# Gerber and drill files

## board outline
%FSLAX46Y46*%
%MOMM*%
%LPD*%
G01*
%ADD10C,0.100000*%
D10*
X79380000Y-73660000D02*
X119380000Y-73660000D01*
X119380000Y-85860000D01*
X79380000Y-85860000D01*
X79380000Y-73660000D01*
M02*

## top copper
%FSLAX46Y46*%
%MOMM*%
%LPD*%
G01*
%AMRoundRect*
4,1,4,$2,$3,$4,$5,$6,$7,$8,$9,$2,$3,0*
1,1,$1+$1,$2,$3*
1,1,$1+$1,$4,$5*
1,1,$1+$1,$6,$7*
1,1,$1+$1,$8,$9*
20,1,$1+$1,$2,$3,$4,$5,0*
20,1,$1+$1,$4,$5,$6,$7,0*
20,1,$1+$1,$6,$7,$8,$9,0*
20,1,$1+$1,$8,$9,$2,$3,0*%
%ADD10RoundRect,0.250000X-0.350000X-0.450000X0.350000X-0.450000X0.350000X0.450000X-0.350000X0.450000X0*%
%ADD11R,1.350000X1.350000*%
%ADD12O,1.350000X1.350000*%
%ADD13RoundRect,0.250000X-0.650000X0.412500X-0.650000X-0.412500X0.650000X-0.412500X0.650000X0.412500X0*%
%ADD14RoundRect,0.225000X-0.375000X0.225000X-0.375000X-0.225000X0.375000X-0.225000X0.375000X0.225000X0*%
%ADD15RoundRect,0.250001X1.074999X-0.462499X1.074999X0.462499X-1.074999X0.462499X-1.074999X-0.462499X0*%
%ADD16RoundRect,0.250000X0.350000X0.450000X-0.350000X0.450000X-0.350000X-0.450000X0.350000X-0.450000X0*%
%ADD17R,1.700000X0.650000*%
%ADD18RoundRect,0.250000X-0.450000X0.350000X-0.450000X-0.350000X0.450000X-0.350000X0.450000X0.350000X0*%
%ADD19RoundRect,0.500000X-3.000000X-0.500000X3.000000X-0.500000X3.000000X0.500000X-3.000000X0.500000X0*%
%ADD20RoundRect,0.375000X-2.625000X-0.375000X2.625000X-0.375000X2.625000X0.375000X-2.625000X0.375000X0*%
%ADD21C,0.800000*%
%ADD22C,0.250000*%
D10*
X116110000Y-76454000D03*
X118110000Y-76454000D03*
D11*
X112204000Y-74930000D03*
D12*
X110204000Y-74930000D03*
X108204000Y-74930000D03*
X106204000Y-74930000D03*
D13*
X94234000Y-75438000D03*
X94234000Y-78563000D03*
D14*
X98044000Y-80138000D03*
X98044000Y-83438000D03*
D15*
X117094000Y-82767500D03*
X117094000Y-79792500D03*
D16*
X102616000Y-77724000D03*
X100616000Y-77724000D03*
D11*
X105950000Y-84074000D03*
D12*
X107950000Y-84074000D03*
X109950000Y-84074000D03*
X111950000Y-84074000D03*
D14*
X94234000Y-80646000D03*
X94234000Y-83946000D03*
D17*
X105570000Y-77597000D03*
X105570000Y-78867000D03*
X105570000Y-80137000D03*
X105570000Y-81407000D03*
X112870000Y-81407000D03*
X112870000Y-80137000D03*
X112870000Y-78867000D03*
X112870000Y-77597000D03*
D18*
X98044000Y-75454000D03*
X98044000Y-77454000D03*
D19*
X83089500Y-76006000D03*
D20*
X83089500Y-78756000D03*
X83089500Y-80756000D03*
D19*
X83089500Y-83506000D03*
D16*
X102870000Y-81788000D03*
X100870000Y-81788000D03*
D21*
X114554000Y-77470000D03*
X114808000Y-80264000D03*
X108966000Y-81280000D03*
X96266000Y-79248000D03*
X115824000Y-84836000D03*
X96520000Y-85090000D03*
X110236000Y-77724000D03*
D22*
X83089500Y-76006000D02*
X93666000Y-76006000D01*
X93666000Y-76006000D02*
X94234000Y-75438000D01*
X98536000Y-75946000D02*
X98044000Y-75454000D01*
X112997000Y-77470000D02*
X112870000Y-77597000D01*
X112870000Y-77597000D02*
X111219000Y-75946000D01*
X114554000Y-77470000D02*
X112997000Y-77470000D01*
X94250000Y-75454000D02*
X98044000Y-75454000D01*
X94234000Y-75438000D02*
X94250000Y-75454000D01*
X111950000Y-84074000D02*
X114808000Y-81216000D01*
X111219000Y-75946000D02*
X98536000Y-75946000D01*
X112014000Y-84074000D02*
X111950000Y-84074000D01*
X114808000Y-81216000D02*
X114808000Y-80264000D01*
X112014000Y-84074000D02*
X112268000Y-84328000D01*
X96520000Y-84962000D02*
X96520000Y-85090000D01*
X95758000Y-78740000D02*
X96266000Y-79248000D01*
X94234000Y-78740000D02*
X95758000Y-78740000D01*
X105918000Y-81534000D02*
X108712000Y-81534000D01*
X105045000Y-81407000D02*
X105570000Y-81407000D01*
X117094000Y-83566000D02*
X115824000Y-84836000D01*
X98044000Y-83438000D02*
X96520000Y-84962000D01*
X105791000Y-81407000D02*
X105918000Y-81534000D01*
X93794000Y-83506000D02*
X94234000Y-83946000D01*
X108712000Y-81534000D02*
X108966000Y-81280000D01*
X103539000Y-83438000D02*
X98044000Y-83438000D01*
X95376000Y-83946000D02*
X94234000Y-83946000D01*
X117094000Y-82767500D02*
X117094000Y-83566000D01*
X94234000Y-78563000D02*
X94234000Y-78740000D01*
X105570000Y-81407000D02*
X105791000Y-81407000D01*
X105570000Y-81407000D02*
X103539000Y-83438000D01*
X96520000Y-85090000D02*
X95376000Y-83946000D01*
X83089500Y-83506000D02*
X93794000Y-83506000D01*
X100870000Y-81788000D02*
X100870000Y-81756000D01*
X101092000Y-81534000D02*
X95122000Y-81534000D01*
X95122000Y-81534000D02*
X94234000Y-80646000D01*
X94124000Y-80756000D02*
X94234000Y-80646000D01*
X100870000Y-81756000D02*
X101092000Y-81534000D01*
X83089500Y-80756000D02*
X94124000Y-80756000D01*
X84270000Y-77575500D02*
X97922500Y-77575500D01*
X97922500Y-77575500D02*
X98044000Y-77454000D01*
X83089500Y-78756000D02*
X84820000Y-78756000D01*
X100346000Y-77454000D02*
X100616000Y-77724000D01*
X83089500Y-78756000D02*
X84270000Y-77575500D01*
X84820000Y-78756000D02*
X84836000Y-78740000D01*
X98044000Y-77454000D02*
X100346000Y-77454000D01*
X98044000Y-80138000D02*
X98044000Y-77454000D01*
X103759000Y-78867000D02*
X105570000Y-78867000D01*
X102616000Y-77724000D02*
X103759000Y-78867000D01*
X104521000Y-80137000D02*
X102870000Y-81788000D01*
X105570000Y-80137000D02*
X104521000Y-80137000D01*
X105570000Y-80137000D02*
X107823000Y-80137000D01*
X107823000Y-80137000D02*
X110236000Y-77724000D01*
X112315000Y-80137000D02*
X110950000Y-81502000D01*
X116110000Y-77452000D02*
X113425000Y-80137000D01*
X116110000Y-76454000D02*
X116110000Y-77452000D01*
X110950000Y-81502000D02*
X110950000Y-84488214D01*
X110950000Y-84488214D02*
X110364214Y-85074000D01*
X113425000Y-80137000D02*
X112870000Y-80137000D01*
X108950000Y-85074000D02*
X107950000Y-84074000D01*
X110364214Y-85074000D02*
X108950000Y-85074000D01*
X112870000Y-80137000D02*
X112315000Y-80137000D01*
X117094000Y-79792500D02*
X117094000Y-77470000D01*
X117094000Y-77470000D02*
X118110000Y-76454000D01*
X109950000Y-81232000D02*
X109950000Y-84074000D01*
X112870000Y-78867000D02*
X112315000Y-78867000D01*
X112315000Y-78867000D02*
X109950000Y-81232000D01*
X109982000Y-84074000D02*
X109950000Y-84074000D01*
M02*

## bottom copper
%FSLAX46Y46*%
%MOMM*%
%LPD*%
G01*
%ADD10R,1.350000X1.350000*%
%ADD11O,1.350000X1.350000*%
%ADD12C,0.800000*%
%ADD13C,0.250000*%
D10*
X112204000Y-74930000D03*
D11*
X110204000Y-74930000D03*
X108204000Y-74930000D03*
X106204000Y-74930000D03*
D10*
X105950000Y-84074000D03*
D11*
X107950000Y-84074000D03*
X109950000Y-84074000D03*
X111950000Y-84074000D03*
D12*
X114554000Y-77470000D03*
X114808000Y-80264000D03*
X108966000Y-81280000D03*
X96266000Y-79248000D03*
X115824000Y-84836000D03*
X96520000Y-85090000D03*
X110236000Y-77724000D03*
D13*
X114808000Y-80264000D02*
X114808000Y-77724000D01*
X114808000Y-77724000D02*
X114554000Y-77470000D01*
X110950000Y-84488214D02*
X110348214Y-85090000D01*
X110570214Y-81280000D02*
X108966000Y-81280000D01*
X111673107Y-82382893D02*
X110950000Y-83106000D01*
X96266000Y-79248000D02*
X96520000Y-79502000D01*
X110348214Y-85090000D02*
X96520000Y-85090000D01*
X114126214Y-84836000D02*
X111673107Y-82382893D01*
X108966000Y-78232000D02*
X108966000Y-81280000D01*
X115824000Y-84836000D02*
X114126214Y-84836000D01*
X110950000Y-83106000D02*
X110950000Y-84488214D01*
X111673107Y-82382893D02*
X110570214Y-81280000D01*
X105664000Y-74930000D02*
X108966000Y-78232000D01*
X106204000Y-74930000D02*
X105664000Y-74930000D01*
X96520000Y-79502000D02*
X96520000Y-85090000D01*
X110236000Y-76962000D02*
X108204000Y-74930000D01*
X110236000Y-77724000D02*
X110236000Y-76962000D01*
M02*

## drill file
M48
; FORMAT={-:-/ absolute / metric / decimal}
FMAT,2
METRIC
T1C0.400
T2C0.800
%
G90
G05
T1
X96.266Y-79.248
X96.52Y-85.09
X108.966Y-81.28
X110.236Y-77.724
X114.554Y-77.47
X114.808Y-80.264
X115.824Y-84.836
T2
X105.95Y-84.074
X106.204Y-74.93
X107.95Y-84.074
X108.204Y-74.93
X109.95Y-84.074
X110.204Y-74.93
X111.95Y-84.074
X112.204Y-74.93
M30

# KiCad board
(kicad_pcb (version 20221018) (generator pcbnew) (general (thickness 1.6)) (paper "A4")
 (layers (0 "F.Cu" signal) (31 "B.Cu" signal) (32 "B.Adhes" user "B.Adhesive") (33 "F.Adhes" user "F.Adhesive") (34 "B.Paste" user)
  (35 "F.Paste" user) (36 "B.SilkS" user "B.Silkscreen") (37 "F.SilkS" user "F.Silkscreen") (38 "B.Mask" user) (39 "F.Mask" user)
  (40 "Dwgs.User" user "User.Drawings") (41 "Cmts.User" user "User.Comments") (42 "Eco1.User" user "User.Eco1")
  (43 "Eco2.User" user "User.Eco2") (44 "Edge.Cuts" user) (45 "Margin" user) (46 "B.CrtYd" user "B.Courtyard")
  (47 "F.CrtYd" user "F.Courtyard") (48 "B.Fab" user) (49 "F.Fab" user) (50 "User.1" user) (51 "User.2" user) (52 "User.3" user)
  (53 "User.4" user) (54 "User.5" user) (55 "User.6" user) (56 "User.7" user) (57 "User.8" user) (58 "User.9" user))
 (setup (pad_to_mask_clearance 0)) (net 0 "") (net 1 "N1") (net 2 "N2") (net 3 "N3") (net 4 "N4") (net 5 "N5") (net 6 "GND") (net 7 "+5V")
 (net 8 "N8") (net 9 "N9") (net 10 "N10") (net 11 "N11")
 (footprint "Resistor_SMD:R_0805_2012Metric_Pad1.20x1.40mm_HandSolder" (layer "F.Cu") (at 117.11 76.454)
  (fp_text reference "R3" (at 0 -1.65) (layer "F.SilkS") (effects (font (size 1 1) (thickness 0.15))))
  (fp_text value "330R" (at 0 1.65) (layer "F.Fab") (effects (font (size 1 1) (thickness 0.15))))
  (pad "1" smd roundrect (at -1 0) (size 1.2 1.4) (layers "F.Cu" "F.Paste" "F.Mask") (roundrect_rratio 0.208333) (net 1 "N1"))
  (pad "2" smd roundrect (at 1 0) (size 1.2 1.4) (layers "F.Cu" "F.Paste" "F.Mask") (roundrect_rratio 0.208333) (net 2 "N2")))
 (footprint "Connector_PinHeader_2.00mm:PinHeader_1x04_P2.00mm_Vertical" (layer "F.Cu") (at 112.204 74.93 -90)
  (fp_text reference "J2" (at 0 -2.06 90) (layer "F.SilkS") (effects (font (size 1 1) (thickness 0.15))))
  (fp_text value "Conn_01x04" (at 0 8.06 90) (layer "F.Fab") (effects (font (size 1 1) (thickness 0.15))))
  (pad "1" thru_hole rect (at 0 0 270) (size 1.35 1.35) (drill 0.8) (layers "*.Cu" "*.Mask") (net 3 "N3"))
  (pad "2" thru_hole oval (at 0 2 270) (size 1.35 1.35) (drill 0.8) (layers "*.Cu" "*.Mask") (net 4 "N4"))
  (pad "3" thru_hole oval (at 0 4 270) (size 1.35 1.35) (drill 0.8) (layers "*.Cu" "*.Mask") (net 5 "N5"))
  (pad "4" thru_hole oval (at 0 6 270) (size 1.35 1.35) (drill 0.8) (layers "*.Cu" "*.Mask") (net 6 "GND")))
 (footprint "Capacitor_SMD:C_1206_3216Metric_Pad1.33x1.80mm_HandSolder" (layer "F.Cu") (at 94.234 77.0005 -90)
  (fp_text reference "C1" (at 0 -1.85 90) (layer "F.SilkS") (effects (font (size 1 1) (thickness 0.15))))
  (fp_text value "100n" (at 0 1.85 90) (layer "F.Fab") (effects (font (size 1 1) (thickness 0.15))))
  (pad "1" smd roundrect (at -1.5625 0 270) (size 1.325 1.8) (layers "F.Cu" "F.Paste" "F.Mask") (roundrect_rratio 0.188679) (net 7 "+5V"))
  (pad "2" smd roundrect (at 1.5625 0 270) (size 1.325 1.8) (layers "F.Cu" "F.Paste" "F.Mask") (roundrect_rratio 0.188679) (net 6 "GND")))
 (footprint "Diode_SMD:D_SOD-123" (layer "F.Cu") (at 98.044 81.788 -90)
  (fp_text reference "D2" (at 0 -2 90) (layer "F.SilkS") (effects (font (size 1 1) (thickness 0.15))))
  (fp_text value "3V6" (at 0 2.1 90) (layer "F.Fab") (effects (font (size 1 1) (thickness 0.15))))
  (pad "1" smd roundrect (at -1.65 0 270) (size 0.9 1.2) (layers "F.Cu" "F.Paste" "F.Mask") (roundrect_rratio 0.25) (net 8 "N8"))
  (pad "2" smd roundrect (at 1.65 0 270) (size 0.9 1.2) (layers "F.Cu" "F.Paste" "F.Mask") (roundrect_rratio 0.25) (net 6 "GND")))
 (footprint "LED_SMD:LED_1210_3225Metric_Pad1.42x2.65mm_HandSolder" (layer "F.Cu") (at 117.094 81.28 90)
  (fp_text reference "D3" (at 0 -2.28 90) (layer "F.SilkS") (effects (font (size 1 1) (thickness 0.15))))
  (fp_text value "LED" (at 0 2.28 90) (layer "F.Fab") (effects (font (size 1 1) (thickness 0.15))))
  (pad "1" smd roundrect (at -1.4875 0 90) (size 1.425 2.65) (layers "F.Cu" "F.Paste" "F.Mask") (roundrect_rratio 0.175439) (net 6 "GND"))
  (pad "2" smd roundrect (at 1.4875 0 90) (size 1.425 2.65) (layers "F.Cu" "F.Paste" "F.Mask") (roundrect_rratio 0.175439) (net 2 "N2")))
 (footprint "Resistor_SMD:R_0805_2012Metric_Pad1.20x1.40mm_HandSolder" (layer "F.Cu") (at 101.616 77.724 180)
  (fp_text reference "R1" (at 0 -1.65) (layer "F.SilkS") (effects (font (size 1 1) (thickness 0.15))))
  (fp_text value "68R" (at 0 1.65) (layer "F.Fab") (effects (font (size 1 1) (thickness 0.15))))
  (pad "1" smd roundrect (at -1 0 180) (size 1.2 1.4) (layers "F.Cu" "F.Paste" "F.Mask") (roundrect_rratio 0.208333) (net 4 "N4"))
  (pad "2" smd roundrect (at 1 0 180) (size 1.2 1.4) (layers "F.Cu" "F.Paste" "F.Mask") (roundrect_rratio 0.208333) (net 8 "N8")))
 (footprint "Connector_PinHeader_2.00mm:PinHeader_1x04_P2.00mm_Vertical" (layer "F.Cu") (at 105.95 84.074 90)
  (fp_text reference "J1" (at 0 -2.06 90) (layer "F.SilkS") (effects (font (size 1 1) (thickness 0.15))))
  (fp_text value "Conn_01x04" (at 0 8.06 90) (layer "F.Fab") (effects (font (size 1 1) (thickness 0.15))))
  (pad "1" thru_hole rect (at 0 0 90) (size 1.35 1.35) (drill 0.8) (layers "*.Cu" "*.Mask") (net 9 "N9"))
  (pad "2" thru_hole oval (at 0 2 90) (size 1.35 1.35) (drill 0.8) (layers "*.Cu" "*.Mask") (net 1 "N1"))
  (pad "3" thru_hole oval (at 0 4 90) (size 1.35 1.35) (drill 0.8) (layers "*.Cu" "*.Mask") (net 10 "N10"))
  (pad "4" thru_hole oval (at 0 6 90) (size 1.35 1.35) (drill 0.8) (layers "*.Cu" "*.Mask") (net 7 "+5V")))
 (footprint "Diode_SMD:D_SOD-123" (layer "F.Cu") (at 94.234 82.296 -90)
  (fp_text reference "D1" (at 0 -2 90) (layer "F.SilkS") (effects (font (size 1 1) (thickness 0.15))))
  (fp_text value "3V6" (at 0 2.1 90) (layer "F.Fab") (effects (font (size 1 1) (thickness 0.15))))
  (pad "1" smd roundrect (at -1.65 0 270) (size 0.9 1.2) (layers "F.Cu" "F.Paste" "F.Mask") (roundrect_rratio 0.25) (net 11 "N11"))
  (pad "2" smd roundrect (at 1.65 0 270) (size 0.9 1.2) (layers "F.Cu" "F.Paste" "F.Mask") (roundrect_rratio 0.25) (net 6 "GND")))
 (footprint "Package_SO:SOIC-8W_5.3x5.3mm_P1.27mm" (layer "F.Cu") (at 109.22 79.502)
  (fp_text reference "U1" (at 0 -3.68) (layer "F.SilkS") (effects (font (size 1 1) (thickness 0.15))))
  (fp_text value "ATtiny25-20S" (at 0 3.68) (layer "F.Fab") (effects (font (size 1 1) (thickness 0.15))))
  (pad "1" smd rect (at -3.65 -1.905) (size 1.7 0.65) (layers "F.Cu" "F.Paste" "F.Mask") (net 3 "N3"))
  (pad "2" smd rect (at -3.65 -0.635) (size 1.7 0.65) (layers "F.Cu" "F.Paste" "F.Mask") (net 4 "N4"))
  (pad "3" smd rect (at -3.65 0.635) (size 1.7 0.65) (layers "F.Cu" "F.Paste" "F.Mask") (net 5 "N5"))
  (pad "4" smd rect (at -3.65 1.905) (size 1.7 0.65) (layers "F.Cu" "F.Paste" "F.Mask") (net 6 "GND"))
  (pad "5" smd rect (at 3.65 1.905) (size 1.7 0.65) (layers "F.Cu" "F.Paste" "F.Mask") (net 9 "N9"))
  (pad "6" smd rect (at 3.65 0.635) (size 1.7 0.65) (layers "F.Cu" "F.Paste" "F.Mask") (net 1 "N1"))
  (pad "7" smd rect (at 3.65 -0.635) (size 1.7 0.65) (layers "F.Cu" "F.Paste" "F.Mask") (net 10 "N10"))
  (pad "8" smd rect (at 3.65 -1.905) (size 1.7 0.65) (layers "F.Cu" "F.Paste" "F.Mask") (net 7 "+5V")))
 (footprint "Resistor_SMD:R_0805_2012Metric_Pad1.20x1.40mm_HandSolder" (layer "F.Cu") (at 98.044 76.454 -90)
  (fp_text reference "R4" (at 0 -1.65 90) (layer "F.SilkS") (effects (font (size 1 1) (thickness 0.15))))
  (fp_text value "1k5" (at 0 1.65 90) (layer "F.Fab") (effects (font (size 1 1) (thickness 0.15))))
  (pad "1" smd roundrect (at -1 0 270) (size 1.2 1.4) (layers "F.Cu" "F.Paste" "F.Mask") (roundrect_rratio 0.208333) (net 7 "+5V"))
  (pad "2" smd roundrect (at 1 0 270) (size 1.2 1.4) (layers "F.Cu" "F.Paste" "F.Mask") (roundrect_rratio 0.208333) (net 8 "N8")))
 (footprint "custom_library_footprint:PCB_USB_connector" (layer "F.Cu") (at 83.0895 79.756)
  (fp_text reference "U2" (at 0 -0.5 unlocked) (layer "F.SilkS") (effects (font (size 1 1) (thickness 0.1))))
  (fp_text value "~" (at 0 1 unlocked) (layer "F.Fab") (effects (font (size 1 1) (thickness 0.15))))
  (pad "1" smd roundrect (at 0 -3.75) (size 7 2) (layers "F.Cu" "F.Paste" "F.Mask") (roundrect_rratio 0.25) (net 7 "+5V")
   (thermal_bridge_angle 45))
  (pad "2" smd roundrect (at 0 -1) (size 6 1.5) (layers "F.Cu" "F.Paste" "F.Mask") (roundrect_rratio 0.25) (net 8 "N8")
   (thermal_bridge_angle 45))
  (pad "3" smd roundrect (at 0 1) (size 6 1.5) (layers "F.Cu" "F.Paste" "F.Mask") (roundrect_rratio 0.25) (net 11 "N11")
   (thermal_bridge_angle 45))
  (pad "4" smd roundrect (at 0 3.75) (size 7 2) (layers "F.Cu" "F.Paste" "F.Mask") (roundrect_rratio 0.25) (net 6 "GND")
   (thermal_bridge_angle 45)))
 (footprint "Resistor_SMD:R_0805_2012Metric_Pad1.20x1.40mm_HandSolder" (layer "F.Cu") (at 101.87 81.788 180)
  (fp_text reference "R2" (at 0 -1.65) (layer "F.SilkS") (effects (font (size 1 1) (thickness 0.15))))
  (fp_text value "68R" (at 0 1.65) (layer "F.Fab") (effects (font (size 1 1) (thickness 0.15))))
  (pad "1" smd roundrect (at -1 0 180) (size 1.2 1.4) (layers "F.Cu" "F.Paste" "F.Mask") (roundrect_rratio 0.208333) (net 5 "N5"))
  (pad "2" smd roundrect (at 1 0 180) (size 1.2 1.4) (layers "F.Cu" "F.Paste" "F.Mask") (roundrect_rratio 0.208333) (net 11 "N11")))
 (gr_rect (start 79.38 73.66) (end 119.38 85.86) (stroke (width 0.1) (type default)) (fill none) (layer "Edge.Cuts"))
 (segment (start 83.0895 76.006) (end 93.666 76.006) (width 0.25) (layer "F.Cu") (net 7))
 (segment (start 93.666 76.006) (end 94.234 75.438) (width 0.25) (layer "F.Cu") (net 7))
 (segment (start 98.536 75.946) (end 98.044 75.454) (width 0.25) (layer "F.Cu") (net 7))
 (segment (start 112.997 77.47) (end 112.87 77.597) (width 0.25) (layer "F.Cu") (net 7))
 (segment (start 112.87 77.597) (end 111.219 75.946) (width 0.25) (layer "F.Cu") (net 7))
 (segment (start 114.554 77.47) (end 112.997 77.47) (width 0.25) (layer "F.Cu") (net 7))
 (segment (start 94.25 75.454) (end 98.044 75.454) (width 0.25) (layer "F.Cu") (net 7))
 (segment (start 94.234 75.438) (end 94.25 75.454) (width 0.25) (layer "F.Cu") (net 7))
 (segment (start 111.95 84.074) (end 114.808 81.216) (width 0.25) (layer "F.Cu") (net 7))
 (segment (start 111.219 75.946) (end 98.536 75.946) (width 0.25) (layer "F.Cu") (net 7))
 (segment (start 112.014 84.074) (end 111.95 84.074) (width 0.25) (layer "F.Cu") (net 7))
 (segment (start 114.808 81.216) (end 114.808 80.264) (width 0.25) (layer "F.Cu") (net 7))
 (segment (start 112.014 84.074) (end 112.268 84.328) (width 0.25) (layer "F.Cu") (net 7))
 (via (at 114.554 77.47) (size 0.8) (drill 0.4) (layers "F.Cu" "B.Cu") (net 7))
 (via (at 114.808 80.264) (size 0.8) (drill 0.4) (layers "F.Cu" "B.Cu") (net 7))
 (segment (start 114.808 80.264) (end 114.808 77.724) (width 0.25) (layer "B.Cu") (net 7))
 (segment (start 114.808 77.724) (end 114.554 77.47) (width 0.25) (layer "B.Cu") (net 7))
 (segment (start 96.52 84.962) (end 96.52 85.09) (width 0.25) (layer "F.Cu") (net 6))
 (segment (start 95.758 78.74) (end 96.266 79.248) (width 0.25) (layer "F.Cu") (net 6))
 (segment (start 94.234 78.74) (end 95.758 78.74) (width 0.25) (layer "F.Cu") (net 6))
 (segment (start 105.918 81.534) (end 108.712 81.534) (width 0.25) (layer "F.Cu") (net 6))
 (segment (start 105.045 81.407) (end 105.57 81.407) (width 0.25) (layer "F.Cu") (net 6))
 (segment (start 117.094 83.566) (end 115.824 84.836) (width 0.25) (layer "F.Cu") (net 6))
 (segment (start 98.044 83.438) (end 96.52 84.962) (width 0.25) (layer "F.Cu") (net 6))
 (segment (start 105.791 81.407) (end 105.918 81.534) (width 0.25) (layer "F.Cu") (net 6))
 (segment (start 93.794 83.506) (end 94.234 83.946) (width 0.25) (layer "F.Cu") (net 6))
 (segment (start 108.712 81.534) (end 108.966 81.28) (width 0.25) (layer "F.Cu") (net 6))
 (segment (start 103.539 83.438) (end 98.044 83.438) (width 0.25) (layer "F.Cu") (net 6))
 (segment (start 95.376 83.946) (end 94.234 83.946) (width 0.25) (layer "F.Cu") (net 6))
 (segment (start 117.094 82.7675) (end 117.094 83.566) (width 0.25) (layer "F.Cu") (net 6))
 (segment (start 94.234 78.563) (end 94.234 78.74) (width 0.25) (layer "F.Cu") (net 6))
 (segment (start 105.57 81.407) (end 105.791 81.407) (width 0.25) (layer "F.Cu") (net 6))
 (segment (start 105.57 81.407) (end 103.539 83.438) (width 0.25) (layer "F.Cu") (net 6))
 (segment (start 96.52 85.09) (end 95.376 83.946) (width 0.25) (layer "F.Cu") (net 6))
 (segment (start 83.0895 83.506) (end 93.794 83.506) (width 0.25) (layer "F.Cu") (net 6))
 (via (at 108.966 81.28) (size 0.8) (drill 0.4) (layers "F.Cu" "B.Cu") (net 6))
 (via (at 96.266 79.248) (size 0.8) (drill 0.4) (layers "F.Cu" "B.Cu") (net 6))
 (via (at 115.824 84.836) (size 0.8) (drill 0.4) (layers "F.Cu" "B.Cu") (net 6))
 (via (at 96.52 85.09) (size 0.8) (drill 0.4) (layers "F.Cu" "B.Cu") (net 6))
 (segment (start 110.95 84.488214) (end 110.348214 85.09) (width 0.25) (layer "B.Cu") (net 6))
 (segment (start 110.570214 81.28) (end 108.966 81.28) (width 0.25) (layer "B.Cu") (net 6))
 (segment (start 111.673107 82.382893) (end 110.95 83.106) (width 0.25) (layer "B.Cu") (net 6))
 (segment (start 96.266 79.248) (end 96.52 79.502) (width 0.25) (layer "B.Cu") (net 6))
 (segment (start 110.348214 85.09) (end 96.52 85.09) (width 0.25) (layer "B.Cu") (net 6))
 (segment (start 114.126214 84.836) (end 111.673107 82.382893) (width 0.25) (layer "B.Cu") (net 6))
 (segment (start 108.966 78.232) (end 108.966 81.28) (width 0.25) (layer "B.Cu") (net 6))
 (segment (start 115.824 84.836) (end 114.126214 84.836) (width 0.25) (layer "B.Cu") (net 6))
 (segment (start 110.95 83.106) (end 110.95 84.488214) (width 0.25) (layer "B.Cu") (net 6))
 (segment (start 111.673107 82.382893) (end 110.570214 81.28) (width 0.25) (layer "B.Cu") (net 6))
 (segment (start 105.664 74.93) (end 108.966 78.232) (width 0.25) (layer "B.Cu") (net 6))
 (segment (start 106.204 74.93) (end 105.664 74.93) (width 0.25) (layer "B.Cu") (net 6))
 (segment (start 96.52 79.502) (end 96.52 85.09) (width 0.25) (layer "B.Cu") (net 6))
 (segment (start 100.87 81.788) (end 100.87 81.756) (width 0.25) (layer "F.Cu") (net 11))
 (segment (start 101.092 81.534) (end 95.122 81.534) (width 0.25) (layer "F.Cu") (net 11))
 (segment (start 95.122 81.534) (end 94.234 80.646) (width 0.25) (layer "F.Cu") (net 11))
 (segment (start 94.124 80.756) (end 94.234 80.646) (width 0.25) (layer "F.Cu") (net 11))
 (segment (start 100.87 81.756) (end 101.092 81.534) (width 0.25) (layer "F.Cu") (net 11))
 (segment (start 83.0895 80.756) (end 94.124 80.756) (width 0.25) (layer "F.Cu") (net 11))
 (segment (start 84.27 77.5755) (end 97.9225 77.5755) (width 0.25) (layer "F.Cu") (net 8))
 (segment (start 97.9225 77.5755) (end 98.044 77.454) (width 0.25) (layer "F.Cu") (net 8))
 (segment (start 83.0895 78.756) (end 84.82 78.756) (width 0.25) (layer "F.Cu") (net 8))
 (segment (start 100.346 77.454) (end 100.616 77.724) (width 0.25) (layer "F.Cu") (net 8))
 (segment (start 83.0895 78.756) (end 84.27 77.5755) (width 0.25) (layer "F.Cu") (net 8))
 (segment (start 84.82 78.756) (end 84.836 78.74) (width 0.25) (layer "F.Cu") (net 8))
 (segment (start 98.044 77.454) (end 100.346 77.454) (width 0.25) (layer "F.Cu") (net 8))
 (segment (start 98.044 80.138) (end 98.044 77.454) (width 0.25) (layer "F.Cu") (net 8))
 (segment (start 103.759 78.867) (end 105.57 78.867) (width 0.25) (layer "F.Cu") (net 4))
 (segment (start 102.616 77.724) (end 103.759 78.867) (width 0.25) (layer "F.Cu") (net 4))
 (segment (start 104.521 80.137) (end 102.87 81.788) (width 0.25) (layer "F.Cu") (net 5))
 (segment (start 105.57 80.137) (end 104.521 80.137) (width 0.25) (layer "F.Cu") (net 5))
 (segment (start 105.57 80.137) (end 107.823 80.137) (width 0.25) (layer "F.Cu") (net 5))
 (segment (start 107.823 80.137) (end 110.236 77.724) (width 0.25) (layer "F.Cu") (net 5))
 (via (at 110.236 77.724) (size 0.8) (drill 0.4) (layers "F.Cu" "B.Cu") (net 5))
 (segment (start 110.236 76.962) (end 108.204 74.93) (width 0.25) (layer "B.Cu") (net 5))
 (segment (start 110.236 77.724) (end 110.236 76.962) (width 0.25) (layer "B.Cu") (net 5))
 (segment (start 112.315 80.137) (end 110.95 81.502) (width 0.25) (layer "F.Cu") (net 1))
 (segment (start 116.11 77.452) (end 113.425 80.137) (width 0.25) (layer "F.Cu") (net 1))
 (segment (start 116.11 76.454) (end 116.11 77.452) (width 0.25) (layer "F.Cu") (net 1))
 (segment (start 110.95 81.502) (end 110.95 84.488214) (width 0.25) (layer "F.Cu") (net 1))
 (segment (start 110.95 84.488214) (end 110.364214 85.074) (width 0.25) (layer "F.Cu") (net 1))
 (segment (start 113.425 80.137) (end 112.87 80.137) (width 0.25) (layer "F.Cu") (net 1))
 (segment (start 108.95 85.074) (end 107.95 84.074) (width 0.25) (layer "F.Cu") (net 1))
 (segment (start 110.364214 85.074) (end 108.95 85.074) (width 0.25) (layer "F.Cu") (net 1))
 (segment (start 112.87 80.137) (end 112.315 80.137) (width 0.25) (layer "F.Cu") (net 1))
 (segment (start 117.094 79.7925) (end 117.094 77.47) (width 0.25) (layer "F.Cu") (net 2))
 (segment (start 117.094 77.47) (end 118.11 76.454) (width 0.25) (layer "F.Cu") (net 2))
 (segment (start 109.95 81.232) (end 109.95 84.074) (width 0.25) (layer "F.Cu") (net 10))
 (segment (start 112.87 78.867) (end 112.315 78.867) (width 0.25) (layer "F.Cu") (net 10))
 (segment (start 112.315 78.867) (end 109.95 81.232) (width 0.25) (layer "F.Cu") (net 10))
 (segment (start 109.982 84.074) (end 109.95 84.074) (width 0.25) (layer "F.Cu") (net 10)))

